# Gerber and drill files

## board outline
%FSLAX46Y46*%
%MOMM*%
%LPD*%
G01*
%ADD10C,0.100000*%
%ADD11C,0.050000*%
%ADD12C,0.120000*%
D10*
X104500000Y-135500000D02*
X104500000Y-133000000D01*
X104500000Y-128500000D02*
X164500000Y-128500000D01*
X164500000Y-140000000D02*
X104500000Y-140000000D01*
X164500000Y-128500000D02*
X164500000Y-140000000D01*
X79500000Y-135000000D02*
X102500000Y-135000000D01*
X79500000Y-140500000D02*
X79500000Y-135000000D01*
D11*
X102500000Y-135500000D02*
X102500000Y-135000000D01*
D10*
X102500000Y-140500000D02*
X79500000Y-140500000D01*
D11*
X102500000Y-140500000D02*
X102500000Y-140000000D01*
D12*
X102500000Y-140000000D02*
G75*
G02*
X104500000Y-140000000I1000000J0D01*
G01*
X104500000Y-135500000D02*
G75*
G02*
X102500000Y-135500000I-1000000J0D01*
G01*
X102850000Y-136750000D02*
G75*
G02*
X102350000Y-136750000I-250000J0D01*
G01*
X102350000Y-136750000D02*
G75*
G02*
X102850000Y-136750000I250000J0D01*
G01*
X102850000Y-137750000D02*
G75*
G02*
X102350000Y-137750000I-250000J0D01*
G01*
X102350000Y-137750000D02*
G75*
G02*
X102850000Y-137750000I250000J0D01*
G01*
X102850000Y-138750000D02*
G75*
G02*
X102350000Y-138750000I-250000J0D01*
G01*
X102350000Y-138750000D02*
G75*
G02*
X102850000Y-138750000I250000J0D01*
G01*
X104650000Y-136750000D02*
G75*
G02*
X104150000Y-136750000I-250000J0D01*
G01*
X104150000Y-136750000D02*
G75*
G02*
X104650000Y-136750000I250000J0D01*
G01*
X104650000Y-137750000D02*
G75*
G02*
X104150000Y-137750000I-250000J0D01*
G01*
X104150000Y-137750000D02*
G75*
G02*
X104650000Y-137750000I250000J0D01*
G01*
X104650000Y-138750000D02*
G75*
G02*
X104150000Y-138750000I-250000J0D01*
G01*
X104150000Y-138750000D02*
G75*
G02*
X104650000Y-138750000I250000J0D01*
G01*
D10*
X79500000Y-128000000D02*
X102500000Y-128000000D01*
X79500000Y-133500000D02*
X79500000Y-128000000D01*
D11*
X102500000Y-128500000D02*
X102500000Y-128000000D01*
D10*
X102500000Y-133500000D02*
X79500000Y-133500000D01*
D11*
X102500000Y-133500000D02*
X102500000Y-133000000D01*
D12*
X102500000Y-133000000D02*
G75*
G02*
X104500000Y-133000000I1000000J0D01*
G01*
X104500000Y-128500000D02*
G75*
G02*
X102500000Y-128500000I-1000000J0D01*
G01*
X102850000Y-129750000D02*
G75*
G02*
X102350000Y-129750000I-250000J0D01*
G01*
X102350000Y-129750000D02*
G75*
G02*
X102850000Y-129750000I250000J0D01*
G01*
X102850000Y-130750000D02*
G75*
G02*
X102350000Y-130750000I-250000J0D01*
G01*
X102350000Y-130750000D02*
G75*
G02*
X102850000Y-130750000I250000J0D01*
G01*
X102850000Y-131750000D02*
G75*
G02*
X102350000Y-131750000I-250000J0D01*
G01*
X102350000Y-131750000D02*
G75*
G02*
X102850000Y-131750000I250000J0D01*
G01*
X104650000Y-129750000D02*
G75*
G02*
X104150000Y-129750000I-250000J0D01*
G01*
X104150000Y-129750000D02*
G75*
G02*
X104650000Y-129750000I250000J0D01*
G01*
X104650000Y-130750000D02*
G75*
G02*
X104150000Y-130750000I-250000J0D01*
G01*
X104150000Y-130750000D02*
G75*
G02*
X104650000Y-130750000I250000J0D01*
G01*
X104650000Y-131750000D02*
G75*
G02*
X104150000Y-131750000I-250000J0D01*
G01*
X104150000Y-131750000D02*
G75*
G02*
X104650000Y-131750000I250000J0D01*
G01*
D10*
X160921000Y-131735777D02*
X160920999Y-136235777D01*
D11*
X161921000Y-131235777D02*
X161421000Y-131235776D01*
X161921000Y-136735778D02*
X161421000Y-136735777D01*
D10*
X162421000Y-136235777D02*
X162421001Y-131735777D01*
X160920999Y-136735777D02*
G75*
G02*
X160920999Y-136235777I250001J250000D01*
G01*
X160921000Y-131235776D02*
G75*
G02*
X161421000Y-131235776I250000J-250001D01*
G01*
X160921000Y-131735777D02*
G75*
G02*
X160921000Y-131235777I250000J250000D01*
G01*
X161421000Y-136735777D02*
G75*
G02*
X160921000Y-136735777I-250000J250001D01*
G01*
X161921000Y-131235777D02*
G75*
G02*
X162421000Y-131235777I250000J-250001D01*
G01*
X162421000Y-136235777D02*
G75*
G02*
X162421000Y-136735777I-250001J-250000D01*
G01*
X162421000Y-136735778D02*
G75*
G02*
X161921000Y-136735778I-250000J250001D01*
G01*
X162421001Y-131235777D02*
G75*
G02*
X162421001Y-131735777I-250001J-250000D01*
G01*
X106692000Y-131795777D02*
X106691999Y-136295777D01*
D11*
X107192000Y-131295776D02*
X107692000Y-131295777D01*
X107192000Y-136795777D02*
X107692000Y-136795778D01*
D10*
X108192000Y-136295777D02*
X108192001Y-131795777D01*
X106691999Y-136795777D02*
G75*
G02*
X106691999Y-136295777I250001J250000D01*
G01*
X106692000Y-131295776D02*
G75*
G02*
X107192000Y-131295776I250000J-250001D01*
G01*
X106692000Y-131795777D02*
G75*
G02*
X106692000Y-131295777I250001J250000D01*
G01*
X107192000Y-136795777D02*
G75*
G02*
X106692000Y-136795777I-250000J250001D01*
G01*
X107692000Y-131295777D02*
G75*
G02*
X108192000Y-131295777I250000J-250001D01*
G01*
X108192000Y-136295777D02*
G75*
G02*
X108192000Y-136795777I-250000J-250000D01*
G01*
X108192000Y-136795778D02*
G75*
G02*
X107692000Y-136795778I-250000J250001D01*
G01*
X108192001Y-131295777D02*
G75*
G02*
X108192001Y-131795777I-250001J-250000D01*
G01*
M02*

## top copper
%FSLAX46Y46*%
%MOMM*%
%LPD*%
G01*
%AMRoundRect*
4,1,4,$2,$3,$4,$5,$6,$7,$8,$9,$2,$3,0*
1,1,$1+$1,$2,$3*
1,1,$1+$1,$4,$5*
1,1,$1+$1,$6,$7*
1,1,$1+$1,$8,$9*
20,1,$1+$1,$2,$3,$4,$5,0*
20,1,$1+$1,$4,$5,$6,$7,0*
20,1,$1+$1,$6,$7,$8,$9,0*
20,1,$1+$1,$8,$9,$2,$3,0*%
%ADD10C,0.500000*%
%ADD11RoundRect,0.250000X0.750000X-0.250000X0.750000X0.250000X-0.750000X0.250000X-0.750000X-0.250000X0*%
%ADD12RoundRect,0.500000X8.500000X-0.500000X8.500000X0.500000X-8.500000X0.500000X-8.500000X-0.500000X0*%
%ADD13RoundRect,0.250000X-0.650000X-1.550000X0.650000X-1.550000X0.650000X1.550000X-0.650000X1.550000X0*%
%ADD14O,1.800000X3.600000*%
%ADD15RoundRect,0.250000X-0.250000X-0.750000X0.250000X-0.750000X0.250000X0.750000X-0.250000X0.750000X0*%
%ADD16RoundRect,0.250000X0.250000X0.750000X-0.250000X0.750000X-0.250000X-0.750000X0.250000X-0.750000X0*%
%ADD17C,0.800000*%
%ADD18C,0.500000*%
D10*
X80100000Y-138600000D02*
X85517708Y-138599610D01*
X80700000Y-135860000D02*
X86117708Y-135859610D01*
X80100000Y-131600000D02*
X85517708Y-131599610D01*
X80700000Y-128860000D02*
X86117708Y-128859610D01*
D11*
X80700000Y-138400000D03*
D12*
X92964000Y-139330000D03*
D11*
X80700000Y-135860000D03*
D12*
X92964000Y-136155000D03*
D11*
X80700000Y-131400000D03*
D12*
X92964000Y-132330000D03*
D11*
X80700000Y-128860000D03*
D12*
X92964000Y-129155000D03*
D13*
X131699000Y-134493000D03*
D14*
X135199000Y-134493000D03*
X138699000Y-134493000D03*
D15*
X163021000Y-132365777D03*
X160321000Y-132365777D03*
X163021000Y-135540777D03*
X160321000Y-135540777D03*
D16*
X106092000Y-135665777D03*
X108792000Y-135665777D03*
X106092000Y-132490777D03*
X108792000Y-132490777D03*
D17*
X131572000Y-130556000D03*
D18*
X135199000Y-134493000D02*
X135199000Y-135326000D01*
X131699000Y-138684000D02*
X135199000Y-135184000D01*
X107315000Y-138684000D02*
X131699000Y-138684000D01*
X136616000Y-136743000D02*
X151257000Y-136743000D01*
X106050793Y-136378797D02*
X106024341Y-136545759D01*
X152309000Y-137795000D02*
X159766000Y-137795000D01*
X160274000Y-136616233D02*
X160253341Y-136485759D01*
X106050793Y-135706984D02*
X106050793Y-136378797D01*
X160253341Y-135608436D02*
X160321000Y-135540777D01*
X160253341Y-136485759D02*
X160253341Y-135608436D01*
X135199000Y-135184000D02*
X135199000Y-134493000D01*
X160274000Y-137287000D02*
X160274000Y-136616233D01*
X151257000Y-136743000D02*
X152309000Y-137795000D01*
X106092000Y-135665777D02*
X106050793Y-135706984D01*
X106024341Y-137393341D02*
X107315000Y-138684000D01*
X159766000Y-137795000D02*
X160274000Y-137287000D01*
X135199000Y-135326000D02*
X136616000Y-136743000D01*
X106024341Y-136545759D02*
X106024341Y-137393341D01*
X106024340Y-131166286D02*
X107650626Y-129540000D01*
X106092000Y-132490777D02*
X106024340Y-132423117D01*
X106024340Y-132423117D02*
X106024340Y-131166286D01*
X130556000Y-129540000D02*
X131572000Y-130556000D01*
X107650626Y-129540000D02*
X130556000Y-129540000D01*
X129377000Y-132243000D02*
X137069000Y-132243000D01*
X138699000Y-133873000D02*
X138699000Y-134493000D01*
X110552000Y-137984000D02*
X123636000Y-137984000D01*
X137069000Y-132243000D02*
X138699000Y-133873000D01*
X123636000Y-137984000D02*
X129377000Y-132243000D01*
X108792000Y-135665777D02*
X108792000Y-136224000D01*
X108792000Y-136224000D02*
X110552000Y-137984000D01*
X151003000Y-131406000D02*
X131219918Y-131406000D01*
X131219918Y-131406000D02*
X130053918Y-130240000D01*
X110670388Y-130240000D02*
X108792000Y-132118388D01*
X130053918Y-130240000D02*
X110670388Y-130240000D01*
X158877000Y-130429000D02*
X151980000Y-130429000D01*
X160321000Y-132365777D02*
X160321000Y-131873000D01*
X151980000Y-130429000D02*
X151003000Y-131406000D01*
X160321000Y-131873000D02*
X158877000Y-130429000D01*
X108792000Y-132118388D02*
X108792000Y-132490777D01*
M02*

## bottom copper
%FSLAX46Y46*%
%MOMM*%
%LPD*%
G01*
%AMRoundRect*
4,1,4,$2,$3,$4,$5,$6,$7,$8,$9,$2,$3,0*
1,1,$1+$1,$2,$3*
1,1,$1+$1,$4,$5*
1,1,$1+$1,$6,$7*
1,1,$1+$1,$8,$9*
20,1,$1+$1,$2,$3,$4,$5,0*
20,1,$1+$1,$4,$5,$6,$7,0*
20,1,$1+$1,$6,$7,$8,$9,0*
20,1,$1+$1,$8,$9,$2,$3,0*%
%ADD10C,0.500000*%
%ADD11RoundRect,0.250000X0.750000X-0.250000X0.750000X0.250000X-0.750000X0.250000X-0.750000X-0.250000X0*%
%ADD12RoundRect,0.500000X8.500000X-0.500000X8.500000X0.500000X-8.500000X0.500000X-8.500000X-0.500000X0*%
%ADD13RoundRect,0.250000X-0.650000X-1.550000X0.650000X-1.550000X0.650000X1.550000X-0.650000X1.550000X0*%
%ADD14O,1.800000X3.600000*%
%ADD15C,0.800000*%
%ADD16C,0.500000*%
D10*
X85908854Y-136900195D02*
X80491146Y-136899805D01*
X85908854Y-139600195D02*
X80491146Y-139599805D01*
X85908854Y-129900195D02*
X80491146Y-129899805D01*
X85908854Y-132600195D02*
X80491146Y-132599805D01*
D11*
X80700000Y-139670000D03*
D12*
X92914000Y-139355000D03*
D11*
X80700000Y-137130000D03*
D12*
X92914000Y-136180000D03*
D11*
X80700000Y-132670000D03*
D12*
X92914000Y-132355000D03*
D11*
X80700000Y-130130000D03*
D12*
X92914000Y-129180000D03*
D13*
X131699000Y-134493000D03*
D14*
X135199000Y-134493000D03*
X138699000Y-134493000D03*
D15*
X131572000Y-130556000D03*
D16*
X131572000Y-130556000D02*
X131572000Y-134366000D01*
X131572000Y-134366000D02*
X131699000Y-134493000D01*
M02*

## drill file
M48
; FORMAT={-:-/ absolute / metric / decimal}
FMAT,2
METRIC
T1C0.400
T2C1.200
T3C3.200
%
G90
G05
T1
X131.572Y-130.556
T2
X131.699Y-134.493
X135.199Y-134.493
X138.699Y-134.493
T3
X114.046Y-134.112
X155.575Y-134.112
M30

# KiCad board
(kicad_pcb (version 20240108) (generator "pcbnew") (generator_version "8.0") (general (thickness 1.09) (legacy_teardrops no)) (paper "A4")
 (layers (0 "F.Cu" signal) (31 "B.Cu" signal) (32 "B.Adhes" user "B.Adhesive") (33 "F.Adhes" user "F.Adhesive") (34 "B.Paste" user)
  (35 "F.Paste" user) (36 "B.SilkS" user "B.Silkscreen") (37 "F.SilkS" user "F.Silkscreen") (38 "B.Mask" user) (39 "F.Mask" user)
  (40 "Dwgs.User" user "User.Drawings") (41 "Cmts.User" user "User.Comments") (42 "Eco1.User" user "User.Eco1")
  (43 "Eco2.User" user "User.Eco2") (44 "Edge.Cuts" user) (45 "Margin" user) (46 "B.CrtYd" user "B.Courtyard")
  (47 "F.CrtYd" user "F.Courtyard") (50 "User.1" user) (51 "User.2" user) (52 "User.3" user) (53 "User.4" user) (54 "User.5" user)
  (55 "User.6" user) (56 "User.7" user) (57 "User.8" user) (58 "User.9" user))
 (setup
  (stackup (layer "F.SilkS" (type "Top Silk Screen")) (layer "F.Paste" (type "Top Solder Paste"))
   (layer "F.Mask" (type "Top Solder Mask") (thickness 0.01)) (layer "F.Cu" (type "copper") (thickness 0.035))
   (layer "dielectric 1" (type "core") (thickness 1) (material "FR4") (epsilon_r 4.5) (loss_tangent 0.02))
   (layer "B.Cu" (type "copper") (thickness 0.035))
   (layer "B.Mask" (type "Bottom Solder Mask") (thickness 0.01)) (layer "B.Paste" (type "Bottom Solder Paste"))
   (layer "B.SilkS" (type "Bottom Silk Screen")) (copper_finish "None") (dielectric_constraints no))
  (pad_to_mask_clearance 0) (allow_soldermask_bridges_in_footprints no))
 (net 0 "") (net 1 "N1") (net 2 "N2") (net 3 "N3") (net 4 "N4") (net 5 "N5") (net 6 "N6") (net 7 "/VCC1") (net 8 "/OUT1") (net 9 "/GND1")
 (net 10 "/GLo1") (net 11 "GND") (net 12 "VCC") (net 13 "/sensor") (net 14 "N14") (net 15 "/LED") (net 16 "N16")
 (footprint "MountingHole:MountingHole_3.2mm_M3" (layer "F.Cu") (at 114.046 134.112)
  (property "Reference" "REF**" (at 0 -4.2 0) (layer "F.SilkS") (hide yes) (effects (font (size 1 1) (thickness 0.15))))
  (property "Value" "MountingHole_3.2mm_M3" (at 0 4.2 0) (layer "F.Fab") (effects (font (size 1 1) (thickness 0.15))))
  (pad "" np_thru_hole circle (at 0 0) (size 3.2 3.2) (drill 3.2) (layers "*.Cu" "*.Mask")))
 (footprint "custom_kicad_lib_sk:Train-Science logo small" (layer "F.Cu") (at 147.574 134.239)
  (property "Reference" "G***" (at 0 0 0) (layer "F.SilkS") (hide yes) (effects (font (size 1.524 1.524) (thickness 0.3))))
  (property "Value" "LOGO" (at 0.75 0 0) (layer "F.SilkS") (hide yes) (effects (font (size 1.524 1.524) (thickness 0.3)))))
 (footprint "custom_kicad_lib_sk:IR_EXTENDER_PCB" (layer "F.Cu") (at 104.5 140)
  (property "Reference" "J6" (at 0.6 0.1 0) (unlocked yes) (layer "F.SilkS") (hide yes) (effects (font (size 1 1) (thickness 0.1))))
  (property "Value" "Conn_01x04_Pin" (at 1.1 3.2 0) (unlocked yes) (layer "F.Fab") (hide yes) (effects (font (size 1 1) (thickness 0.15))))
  (fp_line (start -24.4 -1.4) (end -18.982292 -1.40039) (stroke (width 0.5) (type default)) (layer "F.Cu"))
  (fp_line (start -23.8 -4.14) (end -18.382292 -4.14039) (stroke (width 0.5) (type default)) (layer "F.Cu"))
  (fp_line (start -18.591146 -3.099805) (end -24.008854 -3.100195) (stroke (width 0.5) (type default)) (layer "B.Cu"))
  (fp_line (start -18.591146 -0.399805) (end -24.008854 -0.400195) (stroke (width 0.5) (type default)) (layer "B.Cu"))
  (fp_line (start -25 -5) (end -2 -5) (stroke (width 0.1) (type default)) (layer "Edge.Cuts"))
  (fp_line (start -25 0.5) (end -25 -5) (stroke (width 0.1) (type default)) (layer "Edge.Cuts"))
  (fp_line (start -2 -4.5) (end -2 -5) (stroke (width 0.05) (type default)) (layer "Edge.Cuts"))
  (fp_line (start -2 0.5) (end -25 0.5) (stroke (width 0.1) (type default)) (layer "Edge.Cuts"))
  (fp_line (start -2 0.5) (end -2 0) (stroke (width 0.05) (type default)) (layer "Edge.Cuts"))
  (fp_arc (start -2 0) (mid -1 -1) (end 0 0) (stroke (width 0.12) (type solid)) (layer "Edge.Cuts"))
  (fp_arc (start 0 -4.5) (mid -1 -3.5) (end -2 -4.5) (stroke (width 0.12) (type solid)) (layer "Edge.Cuts"))
  (fp_circle (center -1.9 -3.25) (end -1.9 -3.5) (stroke (width 0.12) (type solid)) (fill none) (layer "Edge.Cuts"))
  (fp_circle (center -1.9 -2.25) (end -1.9 -2.5) (stroke (width 0.12) (type solid)) (fill none) (layer "Edge.Cuts"))
  (fp_circle (center -1.9 -1.25) (end -1.9 -1.5) (stroke (width 0.12) (type solid)) (fill none) (layer "Edge.Cuts"))
  (fp_circle (center -0.1 -3.25) (end -0.1 -3.5) (stroke (width 0.12) (type solid)) (fill none) (layer "Edge.Cuts"))
  (fp_circle (center -0.1 -2.25) (end -0.1 -2.5) (stroke (width 0.12) (type solid)) (fill none) (layer "Edge.Cuts"))
  (fp_circle (center -0.1 -1.25) (end -0.1 -1.5) (stroke (width 0.12) (type solid)) (fill none) (layer "Edge.Cuts"))
  (pad "1" smd roundrect (at -23.8 -0.33 90) (size 1 2) (layers "B.Cu" "B.Paste" "B.Mask") (roundrect_rratio 0.25) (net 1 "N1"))
  (pad "1" smd roundrect (at -11.586 -0.645 90) (size 2 18) (layers "B.Cu" "B.Paste" "B.Mask") (roundrect_rratio 0.25) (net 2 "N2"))
  (pad "2" smd roundrect (at -23.8 -1.6 90) (size 1 2) (layers "F.Cu" "F.Paste" "F.Mask") (roundrect_rratio 0.25) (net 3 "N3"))
  (pad "2" smd roundrect (at -11.536 -0.67 90) (size 2 18) (layers "F.Cu" "F.Paste" "F.Mask") (roundrect_rratio 0.25) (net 3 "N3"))
  (pad "3" smd roundrect (at -23.8 -2.87 90) (size 1 2) (layers "B.Cu" "B.Paste" "B.Mask") (roundrect_rratio 0.25) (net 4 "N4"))
  (pad "3" smd roundrect (at -11.586 -3.82 90) (size 2 18) (layers "B.Cu" "B.Paste" "B.Mask") (roundrect_rratio 0.25) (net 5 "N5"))
  (pad "4" smd roundrect (at -23.8 -4.14 90) (size 1 2) (layers "F.Cu" "F.Paste" "F.Mask") (roundrect_rratio 0.25) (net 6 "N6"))
  (pad "4" smd roundrect (at -11.536 -3.845 90) (size 2 18) (layers "F.Cu" "F.Paste" "F.Mask") (roundrect_rratio 0.25) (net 6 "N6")))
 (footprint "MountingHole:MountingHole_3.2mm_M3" (layer "F.Cu") (at 155.575 134.112)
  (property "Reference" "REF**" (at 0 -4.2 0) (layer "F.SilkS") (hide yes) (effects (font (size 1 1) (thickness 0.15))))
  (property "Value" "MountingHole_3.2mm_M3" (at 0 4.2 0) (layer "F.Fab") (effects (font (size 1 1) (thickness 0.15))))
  (pad "" np_thru_hole circle (at 0 0) (size 3.2 3.2) (drill 3.2) (layers "*.Cu" "*.Mask")))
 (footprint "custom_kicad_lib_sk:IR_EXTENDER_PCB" (layer "F.Cu") (at 104.5 133)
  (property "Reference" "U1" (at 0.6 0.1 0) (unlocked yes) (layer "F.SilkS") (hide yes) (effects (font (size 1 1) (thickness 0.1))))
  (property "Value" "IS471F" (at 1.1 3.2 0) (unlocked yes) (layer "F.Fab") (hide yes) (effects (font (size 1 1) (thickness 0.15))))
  (fp_line (start -24.4 -1.4) (end -18.982292 -1.40039) (stroke (width 0.5) (type default)) (layer "F.Cu"))
  (fp_line (start -23.8 -4.14) (end -18.382292 -4.14039) (stroke (width 0.5) (type default)) (layer "F.Cu"))
  (fp_line (start -18.591146 -3.099805) (end -24.008854 -3.100195) (stroke (width 0.5) (type default)) (layer "B.Cu"))
  (fp_line (start -18.591146 -0.399805) (end -24.008854 -0.400195) (stroke (width 0.5) (type default)) (layer "B.Cu"))
  (fp_line (start -25 -5) (end -2 -5) (stroke (width 0.1) (type default)) (layer "Edge.Cuts"))
  (fp_line (start -25 0.5) (end -25 -5) (stroke (width 0.1) (type default)) (layer "Edge.Cuts"))
  (fp_line (start -2 -4.5) (end -2 -5) (stroke (width 0.05) (type default)) (layer "Edge.Cuts"))
  (fp_line (start -2 0.5) (end -25 0.5) (stroke (width 0.1) (type default)) (layer "Edge.Cuts"))
  (fp_line (start -2 0.5) (end -2 0) (stroke (width 0.05) (type default)) (layer "Edge.Cuts"))
  (fp_arc (start -2 0) (mid -1 -1) (end 0 0) (stroke (width 0.12) (type solid)) (layer "Edge.Cuts"))
  (fp_arc (start 0 -4.5) (mid -1 -3.5) (end -2 -4.5) (stroke (width 0.12) (type solid)) (layer "Edge.Cuts"))
  (fp_circle (center -1.9 -3.25) (end -1.9 -3.5) (stroke (width 0.12) (type solid)) (fill none) (layer "Edge.Cuts"))
  (fp_circle (center -1.9 -2.25) (end -1.9 -2.5) (stroke (width 0.12) (type solid)) (fill none) (layer "Edge.Cuts"))
  (fp_circle (center -1.9 -1.25) (end -1.9 -1.5) (stroke (width 0.12) (type solid)) (fill none) (layer "Edge.Cuts"))
  (fp_circle (center -0.1 -3.25) (end -0.1 -3.5) (stroke (width 0.12) (type solid)) (fill none) (layer "Edge.Cuts"))
  (fp_circle (center -0.1 -2.25) (end -0.1 -2.5) (stroke (width 0.12) (type solid)) (fill none) (layer "Edge.Cuts"))
  (fp_circle (center -0.1 -1.25) (end -0.1 -1.5) (stroke (width 0.12) (type solid)) (fill none) (layer "Edge.Cuts"))
  (pad "1" smd roundrect (at -23.8 -0.33 90) (size 1 2) (layers "B.Cu" "B.Paste" "B.Mask") (roundrect_rratio 0.25) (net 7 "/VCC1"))
  (pad "1" smd roundrect (at -11.586 -0.645 90) (size 2 18) (layers "B.Cu" "B.Paste" "B.Mask") (roundrect_rratio 0.25) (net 7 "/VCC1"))
  (pad "2" smd roundrect (at -23.8 -1.6 90) (size 1 2) (layers "F.Cu" "F.Paste" "F.Mask") (roundrect_rratio 0.25) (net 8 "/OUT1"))
  (pad "2" smd roundrect (at -11.536 -0.67 90) (size 2 18) (layers "F.Cu" "F.Paste" "F.Mask") (roundrect_rratio 0.25) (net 8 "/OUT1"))
  (pad "3" smd roundrect (at -23.8 -2.87 90) (size 1 2) (layers "B.Cu" "B.Paste" "B.Mask") (roundrect_rratio 0.25) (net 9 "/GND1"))
  (pad "3" smd roundrect (at -11.586 -3.82 90) (size 2 18) (layers "B.Cu" "B.Paste" "B.Mask") (roundrect_rratio 0.25) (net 9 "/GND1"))
  (pad "4" smd roundrect (at -23.8 -4.14 90) (size 1 2) (layers "F.Cu" "F.Paste" "F.Mask") (roundrect_rratio 0.25) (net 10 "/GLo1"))
  (pad "4" smd roundrect (at -11.536 -3.845 90) (size 2 18) (layers "F.Cu" "F.Paste" "F.Mask") (roundrect_rratio 0.25) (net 10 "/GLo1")))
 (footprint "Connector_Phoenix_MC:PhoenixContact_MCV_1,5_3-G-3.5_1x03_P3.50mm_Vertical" (layer "F.Cu") (at 131.699 134.493)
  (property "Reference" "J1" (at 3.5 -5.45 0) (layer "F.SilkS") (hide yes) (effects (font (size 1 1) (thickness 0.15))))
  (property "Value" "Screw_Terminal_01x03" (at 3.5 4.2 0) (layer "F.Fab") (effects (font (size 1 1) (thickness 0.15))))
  (pad "1" thru_hole roundrect (at 0 0) (size 1.8 3.6) (drill 1.2) (layers "*.Cu" "*.Mask") (remove_unused_layers no)
   (roundrect_rratio 0.138889) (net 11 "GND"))
  (pad "2" thru_hole oval (at 3.5 0) (size 1.8 3.6) (drill 1.2) (layers "*.Cu" "*.Mask") (remove_unused_layers no) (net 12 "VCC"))
  (pad "3" thru_hole oval (at 7 0) (size 1.8 3.6) (drill 1.2) (layers "*.Cu" "*.Mask") (remove_unused_layers no) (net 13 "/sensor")))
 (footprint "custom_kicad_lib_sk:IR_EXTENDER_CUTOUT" (layer "F.Cu") (at 161.671 134.015777 180)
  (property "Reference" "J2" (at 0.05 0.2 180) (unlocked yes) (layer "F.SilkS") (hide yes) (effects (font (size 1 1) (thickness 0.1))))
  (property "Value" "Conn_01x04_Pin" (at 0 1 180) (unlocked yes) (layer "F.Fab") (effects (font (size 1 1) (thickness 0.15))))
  (fp_line (start 0.75 2.28) (end 0.750001 -2.22) (stroke (width 0.1) (type default)) (layer "Edge.Cuts"))
  (fp_line (start -0.25 2.78) (end 0.25 2.780001) (stroke (width 0.05) (type default)) (layer "Edge.Cuts"))
  (fp_line (start -0.25 -2.720001) (end 0.25 -2.72) (stroke (width 0.05) (type default)) (layer "Edge.Cuts"))
  (fp_line (start -0.75 -2.22) (end -0.750001 2.28) (stroke (width 0.1) (type default)) (layer "Edge.Cuts"))
  (fp_arc (start 0.750001 -2.72) (mid 0.853554 -2.47) (end 0.750001 -2.22) (stroke (width 0.1) (type default)) (layer "Edge.Cuts"))
  (fp_arc (start 0.75 2.780001) (mid 0.5 2.883554) (end 0.25 2.780001) (stroke (width 0.1) (type default)) (layer "Edge.Cuts"))
  (fp_arc (start 0.75 2.28) (mid 0.853553 2.53) (end 0.75 2.78) (stroke (width 0.1) (type default)) (layer "Edge.Cuts"))
  (fp_arc (start 0.25 -2.72) (mid 0.5 -2.823553) (end 0.75 -2.72) (stroke (width 0.1) (type default)) (layer "Edge.Cuts"))
  (fp_arc (start -0.25 2.78) (mid -0.5 2.883553) (end -0.75 2.78) (stroke (width 0.1) (type default)) (layer "Edge.Cuts"))
  (fp_arc (start -0.75 -2.22) (mid -0.853553 -2.47) (end -0.75 -2.72) (stroke (width 0.1) (type default)) (layer "Edge.Cuts"))
  (fp_arc (start -0.75 -2.720001) (mid -0.5 -2.823554) (end -0.25 -2.720001) (stroke (width 0.1) (type default)) (layer "Edge.Cuts"))
  (fp_arc (start -0.750001 2.78) (mid -0.853554 2.53) (end -0.750001 2.28) (stroke (width 0.1) (type default)) (layer "Edge.Cuts"))
  (pad "1" smd roundrect (at -1.35 1.65) (size 1 2) (layers "F.Cu" "F.Paste" "F.Mask") (roundrect_rratio 0.25) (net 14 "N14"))
  (pad "2" smd roundrect (at 1.35 1.65) (size 1 2) (layers "F.Cu" "F.Paste" "F.Mask") (roundrect_rratio 0.25) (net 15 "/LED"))
  (pad "3" smd roundrect (at -1.35 -1.525) (size 1 2) (layers "F.Cu" "F.Paste" "F.Mask") (roundrect_rratio 0.25) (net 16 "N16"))
  (pad "4" smd roundrect (at 1.35 -1.525) (size 1 2) (layers "F.Cu" "F.Paste" "F.Mask") (roundrect_rratio 0.25) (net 12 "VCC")))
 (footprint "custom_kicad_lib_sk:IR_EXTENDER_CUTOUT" (layer "F.Cu") (at 107.442 134.015777)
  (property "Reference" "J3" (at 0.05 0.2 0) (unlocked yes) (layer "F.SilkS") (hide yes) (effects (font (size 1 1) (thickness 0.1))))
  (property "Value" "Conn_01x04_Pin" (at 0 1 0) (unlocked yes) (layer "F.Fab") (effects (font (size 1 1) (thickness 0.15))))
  (fp_line (start -0.75 -2.22) (end -0.750001 2.28) (stroke (width 0.1) (type default)) (layer "Edge.Cuts"))
  (fp_line (start -0.25 -2.720001) (end 0.25 -2.72) (stroke (width 0.05) (type default)) (layer "Edge.Cuts"))
  (fp_line (start -0.25 2.78) (end 0.25 2.780001) (stroke (width 0.05) (type default)) (layer "Edge.Cuts"))
  (fp_line (start 0.75 2.28) (end 0.750001 -2.22) (stroke (width 0.1) (type default)) (layer "Edge.Cuts"))
  (fp_arc (start -0.750001 2.78) (mid -0.853554 2.53) (end -0.750001 2.28) (stroke (width 0.1) (type default)) (layer "Edge.Cuts"))
  (fp_arc (start -0.75 -2.720001) (mid -0.5 -2.823554) (end -0.25 -2.720001) (stroke (width 0.1) (type default)) (layer "Edge.Cuts"))
  (fp_arc (start -0.75 -2.22) (mid -0.853553 -2.47) (end -0.75 -2.72) (stroke (width 0.1) (type default)) (layer "Edge.Cuts"))
  (fp_arc (start -0.25 2.78) (mid -0.5 2.883553) (end -0.75 2.78) (stroke (width 0.1) (type default)) (layer "Edge.Cuts"))
  (fp_arc (start 0.25 -2.72) (mid 0.5 -2.823553) (end 0.75 -2.72) (stroke (width 0.1) (type default)) (layer "Edge.Cuts"))
  (fp_arc (start 0.75 2.28) (mid 0.853553 2.53) (end 0.75 2.78) (stroke (width 0.1) (type default)) (layer "Edge.Cuts"))
  (fp_arc (start 0.75 2.780001) (mid 0.5 2.883554) (end 0.25 2.780001) (stroke (width 0.1) (type default)) (layer "Edge.Cuts"))
  (fp_arc (start 0.750001 -2.72) (mid 0.853554 -2.47) (end 0.750001 -2.22) (stroke (width 0.1) (type default)) (layer "Edge.Cuts"))
  (pad "1" smd roundrect (at -1.35 1.65 180) (size 1 2) (layers "F.Cu" "F.Paste" "F.Mask") (roundrect_rratio 0.25) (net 12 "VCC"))
  (pad "2" smd roundrect (at 1.35 1.65 180) (size 1 2) (layers "F.Cu" "F.Paste" "F.Mask") (roundrect_rratio 0.25) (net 13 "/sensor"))
  (pad "3" smd roundrect (at -1.35 -1.525 180) (size 1 2) (layers "F.Cu" "F.Paste" "F.Mask") (roundrect_rratio 0.25) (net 11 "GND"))
  (pad "4" smd roundrect (at 1.35 -1.525 180) (size 1 2) (layers "F.Cu" "F.Paste" "F.Mask") (roundrect_rratio 0.25) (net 15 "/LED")))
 (gr_line (start 104.5 135.5) (end 104.5 133) (stroke (width 0.1) (type default)) (layer "Edge.Cuts"))
 (gr_line (start 104.5 128.5) (end 164.5 128.5) (stroke (width 0.1) (type default)) (layer "Edge.Cuts"))
 (gr_line (start 164.5 140) (end 104.5 140) (stroke (width 0.1) (type default)) (layer "Edge.Cuts"))
 (gr_line (start 164.5 128.5) (end 164.5 140) (stroke (width 0.1) (type default)) (layer "Edge.Cuts"))
 (segment (start 135.199 134.493) (end 135.199 135.326) (width 0.5) (layer "F.Cu") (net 12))
 (segment (start 131.699 138.684) (end 135.199 135.184) (width 0.5) (layer "F.Cu") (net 12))
 (segment (start 107.315 138.684) (end 131.699 138.684) (width 0.5) (layer "F.Cu") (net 12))
 (segment (start 136.616 136.743) (end 151.257 136.743) (width 0.5) (layer "F.Cu") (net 12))
 (segment (start 106.050793 136.378797) (end 106.024341 136.545759) (width 0.5) (layer "F.Cu") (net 12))
 (segment (start 152.309 137.795) (end 159.766 137.795) (width 0.5) (layer "F.Cu") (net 12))
 (segment (start 160.274 136.616233) (end 160.253341 136.485759) (width 0.5) (layer "F.Cu") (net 12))
 (segment (start 106.050793 135.706984) (end 106.050793 136.378797) (width 0.5) (layer "F.Cu") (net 12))
 (segment (start 160.253341 135.608436) (end 160.321 135.540777) (width 0.5) (layer "F.Cu") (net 12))
 (segment (start 160.253341 136.485759) (end 160.253341 135.608436) (width 0.5) (layer "F.Cu") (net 12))
 (segment (start 135.199 135.184) (end 135.199 134.493) (width 0.5) (layer "F.Cu") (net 12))
 (segment (start 160.274 137.287) (end 160.274 136.616233) (width 0.5) (layer "F.Cu") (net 12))
 (segment (start 151.257 136.743) (end 152.309 137.795) (width 0.5) (layer "F.Cu") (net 12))
 (segment (start 106.092 135.665777) (end 106.050793 135.706984) (width 0.5) (layer "F.Cu") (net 12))
 (segment (start 106.024341 137.393341) (end 107.315 138.684) (width 0.5) (layer "F.Cu") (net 12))
 (segment (start 159.766 137.795) (end 160.274 137.287) (width 0.5) (layer "F.Cu") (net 12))
 (segment (start 135.199 135.326) (end 136.616 136.743) (width 0.5) (layer "F.Cu") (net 12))
 (segment (start 106.024341 136.545759) (end 106.024341 137.393341) (width 0.5) (layer "F.Cu") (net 12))
 (segment (start 106.02434 131.166286) (end 107.650626 129.54) (width 0.5) (layer "F.Cu") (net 11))
 (segment (start 106.092 132.490777) (end 106.02434 132.423117) (width 0.5) (layer "F.Cu") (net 11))
 (segment (start 106.02434 132.423117) (end 106.02434 131.166286) (width 0.5) (layer "F.Cu") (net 11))
 (segment (start 130.556 129.54) (end 131.572 130.556) (width 0.5) (layer "F.Cu") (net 11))
 (segment (start 107.650626 129.54) (end 130.556 129.54) (width 0.5) (layer "F.Cu") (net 11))
 (via (at 131.572 130.556) (size 0.8) (drill 0.4) (layers "F.Cu" "B.Cu") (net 11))
 (segment (start 131.572 130.556) (end 131.572 134.366) (width 0.5) (layer "B.Cu") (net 11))
 (segment (start 131.572 134.366) (end 131.699 134.493) (width 0.5) (layer "B.Cu") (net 11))
 (segment (start 129.377 132.243) (end 137.069 132.243) (width 0.5) (layer "F.Cu") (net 13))
 (segment (start 138.699 133.873) (end 138.699 134.493) (width 0.5) (layer "F.Cu") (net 13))
 (segment (start 110.552 137.984) (end 123.636 137.984) (width 0.5) (layer "F.Cu") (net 13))
 (segment (start 137.069 132.243) (end 138.699 133.873) (width 0.5) (layer "F.Cu") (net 13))
 (segment (start 123.636 137.984) (end 129.377 132.243) (width 0.5) (layer "F.Cu") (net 13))
 (segment (start 108.792 135.665777) (end 108.792 136.224) (width 0.5) (layer "F.Cu") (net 13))
 (segment (start 108.792 136.224) (end 110.552 137.984) (width 0.5) (layer "F.Cu") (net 13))
 (segment (start 151.003 131.406) (end 131.219918 131.406) (width 0.5) (layer "F.Cu") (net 15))
 (segment (start 131.219918 131.406) (end 130.053918 130.24) (width 0.5) (layer "F.Cu") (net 15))
 (segment (start 110.670388 130.24) (end 108.792 132.118388) (width 0.5) (layer "F.Cu") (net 15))
 (segment (start 130.053918 130.24) (end 110.670388 130.24) (width 0.5) (layer "F.Cu") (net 15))
 (segment (start 158.877 130.429) (end 151.98 130.429) (width 0.5) (layer "F.Cu") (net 15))
 (segment (start 160.321 132.365777) (end 160.321 131.873) (width 0.5) (layer "F.Cu") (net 15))
 (segment (start 151.98 130.429) (end 151.003 131.406) (width 0.5) (layer "F.Cu") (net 15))
 (segment (start 160.321 131.873) (end 158.877 130.429) (width 0.5) (layer "F.Cu") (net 15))
 (segment (start 108.792 132.118388) (end 108.792 132.490777) (width 0.5) (layer "F.Cu") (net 15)))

